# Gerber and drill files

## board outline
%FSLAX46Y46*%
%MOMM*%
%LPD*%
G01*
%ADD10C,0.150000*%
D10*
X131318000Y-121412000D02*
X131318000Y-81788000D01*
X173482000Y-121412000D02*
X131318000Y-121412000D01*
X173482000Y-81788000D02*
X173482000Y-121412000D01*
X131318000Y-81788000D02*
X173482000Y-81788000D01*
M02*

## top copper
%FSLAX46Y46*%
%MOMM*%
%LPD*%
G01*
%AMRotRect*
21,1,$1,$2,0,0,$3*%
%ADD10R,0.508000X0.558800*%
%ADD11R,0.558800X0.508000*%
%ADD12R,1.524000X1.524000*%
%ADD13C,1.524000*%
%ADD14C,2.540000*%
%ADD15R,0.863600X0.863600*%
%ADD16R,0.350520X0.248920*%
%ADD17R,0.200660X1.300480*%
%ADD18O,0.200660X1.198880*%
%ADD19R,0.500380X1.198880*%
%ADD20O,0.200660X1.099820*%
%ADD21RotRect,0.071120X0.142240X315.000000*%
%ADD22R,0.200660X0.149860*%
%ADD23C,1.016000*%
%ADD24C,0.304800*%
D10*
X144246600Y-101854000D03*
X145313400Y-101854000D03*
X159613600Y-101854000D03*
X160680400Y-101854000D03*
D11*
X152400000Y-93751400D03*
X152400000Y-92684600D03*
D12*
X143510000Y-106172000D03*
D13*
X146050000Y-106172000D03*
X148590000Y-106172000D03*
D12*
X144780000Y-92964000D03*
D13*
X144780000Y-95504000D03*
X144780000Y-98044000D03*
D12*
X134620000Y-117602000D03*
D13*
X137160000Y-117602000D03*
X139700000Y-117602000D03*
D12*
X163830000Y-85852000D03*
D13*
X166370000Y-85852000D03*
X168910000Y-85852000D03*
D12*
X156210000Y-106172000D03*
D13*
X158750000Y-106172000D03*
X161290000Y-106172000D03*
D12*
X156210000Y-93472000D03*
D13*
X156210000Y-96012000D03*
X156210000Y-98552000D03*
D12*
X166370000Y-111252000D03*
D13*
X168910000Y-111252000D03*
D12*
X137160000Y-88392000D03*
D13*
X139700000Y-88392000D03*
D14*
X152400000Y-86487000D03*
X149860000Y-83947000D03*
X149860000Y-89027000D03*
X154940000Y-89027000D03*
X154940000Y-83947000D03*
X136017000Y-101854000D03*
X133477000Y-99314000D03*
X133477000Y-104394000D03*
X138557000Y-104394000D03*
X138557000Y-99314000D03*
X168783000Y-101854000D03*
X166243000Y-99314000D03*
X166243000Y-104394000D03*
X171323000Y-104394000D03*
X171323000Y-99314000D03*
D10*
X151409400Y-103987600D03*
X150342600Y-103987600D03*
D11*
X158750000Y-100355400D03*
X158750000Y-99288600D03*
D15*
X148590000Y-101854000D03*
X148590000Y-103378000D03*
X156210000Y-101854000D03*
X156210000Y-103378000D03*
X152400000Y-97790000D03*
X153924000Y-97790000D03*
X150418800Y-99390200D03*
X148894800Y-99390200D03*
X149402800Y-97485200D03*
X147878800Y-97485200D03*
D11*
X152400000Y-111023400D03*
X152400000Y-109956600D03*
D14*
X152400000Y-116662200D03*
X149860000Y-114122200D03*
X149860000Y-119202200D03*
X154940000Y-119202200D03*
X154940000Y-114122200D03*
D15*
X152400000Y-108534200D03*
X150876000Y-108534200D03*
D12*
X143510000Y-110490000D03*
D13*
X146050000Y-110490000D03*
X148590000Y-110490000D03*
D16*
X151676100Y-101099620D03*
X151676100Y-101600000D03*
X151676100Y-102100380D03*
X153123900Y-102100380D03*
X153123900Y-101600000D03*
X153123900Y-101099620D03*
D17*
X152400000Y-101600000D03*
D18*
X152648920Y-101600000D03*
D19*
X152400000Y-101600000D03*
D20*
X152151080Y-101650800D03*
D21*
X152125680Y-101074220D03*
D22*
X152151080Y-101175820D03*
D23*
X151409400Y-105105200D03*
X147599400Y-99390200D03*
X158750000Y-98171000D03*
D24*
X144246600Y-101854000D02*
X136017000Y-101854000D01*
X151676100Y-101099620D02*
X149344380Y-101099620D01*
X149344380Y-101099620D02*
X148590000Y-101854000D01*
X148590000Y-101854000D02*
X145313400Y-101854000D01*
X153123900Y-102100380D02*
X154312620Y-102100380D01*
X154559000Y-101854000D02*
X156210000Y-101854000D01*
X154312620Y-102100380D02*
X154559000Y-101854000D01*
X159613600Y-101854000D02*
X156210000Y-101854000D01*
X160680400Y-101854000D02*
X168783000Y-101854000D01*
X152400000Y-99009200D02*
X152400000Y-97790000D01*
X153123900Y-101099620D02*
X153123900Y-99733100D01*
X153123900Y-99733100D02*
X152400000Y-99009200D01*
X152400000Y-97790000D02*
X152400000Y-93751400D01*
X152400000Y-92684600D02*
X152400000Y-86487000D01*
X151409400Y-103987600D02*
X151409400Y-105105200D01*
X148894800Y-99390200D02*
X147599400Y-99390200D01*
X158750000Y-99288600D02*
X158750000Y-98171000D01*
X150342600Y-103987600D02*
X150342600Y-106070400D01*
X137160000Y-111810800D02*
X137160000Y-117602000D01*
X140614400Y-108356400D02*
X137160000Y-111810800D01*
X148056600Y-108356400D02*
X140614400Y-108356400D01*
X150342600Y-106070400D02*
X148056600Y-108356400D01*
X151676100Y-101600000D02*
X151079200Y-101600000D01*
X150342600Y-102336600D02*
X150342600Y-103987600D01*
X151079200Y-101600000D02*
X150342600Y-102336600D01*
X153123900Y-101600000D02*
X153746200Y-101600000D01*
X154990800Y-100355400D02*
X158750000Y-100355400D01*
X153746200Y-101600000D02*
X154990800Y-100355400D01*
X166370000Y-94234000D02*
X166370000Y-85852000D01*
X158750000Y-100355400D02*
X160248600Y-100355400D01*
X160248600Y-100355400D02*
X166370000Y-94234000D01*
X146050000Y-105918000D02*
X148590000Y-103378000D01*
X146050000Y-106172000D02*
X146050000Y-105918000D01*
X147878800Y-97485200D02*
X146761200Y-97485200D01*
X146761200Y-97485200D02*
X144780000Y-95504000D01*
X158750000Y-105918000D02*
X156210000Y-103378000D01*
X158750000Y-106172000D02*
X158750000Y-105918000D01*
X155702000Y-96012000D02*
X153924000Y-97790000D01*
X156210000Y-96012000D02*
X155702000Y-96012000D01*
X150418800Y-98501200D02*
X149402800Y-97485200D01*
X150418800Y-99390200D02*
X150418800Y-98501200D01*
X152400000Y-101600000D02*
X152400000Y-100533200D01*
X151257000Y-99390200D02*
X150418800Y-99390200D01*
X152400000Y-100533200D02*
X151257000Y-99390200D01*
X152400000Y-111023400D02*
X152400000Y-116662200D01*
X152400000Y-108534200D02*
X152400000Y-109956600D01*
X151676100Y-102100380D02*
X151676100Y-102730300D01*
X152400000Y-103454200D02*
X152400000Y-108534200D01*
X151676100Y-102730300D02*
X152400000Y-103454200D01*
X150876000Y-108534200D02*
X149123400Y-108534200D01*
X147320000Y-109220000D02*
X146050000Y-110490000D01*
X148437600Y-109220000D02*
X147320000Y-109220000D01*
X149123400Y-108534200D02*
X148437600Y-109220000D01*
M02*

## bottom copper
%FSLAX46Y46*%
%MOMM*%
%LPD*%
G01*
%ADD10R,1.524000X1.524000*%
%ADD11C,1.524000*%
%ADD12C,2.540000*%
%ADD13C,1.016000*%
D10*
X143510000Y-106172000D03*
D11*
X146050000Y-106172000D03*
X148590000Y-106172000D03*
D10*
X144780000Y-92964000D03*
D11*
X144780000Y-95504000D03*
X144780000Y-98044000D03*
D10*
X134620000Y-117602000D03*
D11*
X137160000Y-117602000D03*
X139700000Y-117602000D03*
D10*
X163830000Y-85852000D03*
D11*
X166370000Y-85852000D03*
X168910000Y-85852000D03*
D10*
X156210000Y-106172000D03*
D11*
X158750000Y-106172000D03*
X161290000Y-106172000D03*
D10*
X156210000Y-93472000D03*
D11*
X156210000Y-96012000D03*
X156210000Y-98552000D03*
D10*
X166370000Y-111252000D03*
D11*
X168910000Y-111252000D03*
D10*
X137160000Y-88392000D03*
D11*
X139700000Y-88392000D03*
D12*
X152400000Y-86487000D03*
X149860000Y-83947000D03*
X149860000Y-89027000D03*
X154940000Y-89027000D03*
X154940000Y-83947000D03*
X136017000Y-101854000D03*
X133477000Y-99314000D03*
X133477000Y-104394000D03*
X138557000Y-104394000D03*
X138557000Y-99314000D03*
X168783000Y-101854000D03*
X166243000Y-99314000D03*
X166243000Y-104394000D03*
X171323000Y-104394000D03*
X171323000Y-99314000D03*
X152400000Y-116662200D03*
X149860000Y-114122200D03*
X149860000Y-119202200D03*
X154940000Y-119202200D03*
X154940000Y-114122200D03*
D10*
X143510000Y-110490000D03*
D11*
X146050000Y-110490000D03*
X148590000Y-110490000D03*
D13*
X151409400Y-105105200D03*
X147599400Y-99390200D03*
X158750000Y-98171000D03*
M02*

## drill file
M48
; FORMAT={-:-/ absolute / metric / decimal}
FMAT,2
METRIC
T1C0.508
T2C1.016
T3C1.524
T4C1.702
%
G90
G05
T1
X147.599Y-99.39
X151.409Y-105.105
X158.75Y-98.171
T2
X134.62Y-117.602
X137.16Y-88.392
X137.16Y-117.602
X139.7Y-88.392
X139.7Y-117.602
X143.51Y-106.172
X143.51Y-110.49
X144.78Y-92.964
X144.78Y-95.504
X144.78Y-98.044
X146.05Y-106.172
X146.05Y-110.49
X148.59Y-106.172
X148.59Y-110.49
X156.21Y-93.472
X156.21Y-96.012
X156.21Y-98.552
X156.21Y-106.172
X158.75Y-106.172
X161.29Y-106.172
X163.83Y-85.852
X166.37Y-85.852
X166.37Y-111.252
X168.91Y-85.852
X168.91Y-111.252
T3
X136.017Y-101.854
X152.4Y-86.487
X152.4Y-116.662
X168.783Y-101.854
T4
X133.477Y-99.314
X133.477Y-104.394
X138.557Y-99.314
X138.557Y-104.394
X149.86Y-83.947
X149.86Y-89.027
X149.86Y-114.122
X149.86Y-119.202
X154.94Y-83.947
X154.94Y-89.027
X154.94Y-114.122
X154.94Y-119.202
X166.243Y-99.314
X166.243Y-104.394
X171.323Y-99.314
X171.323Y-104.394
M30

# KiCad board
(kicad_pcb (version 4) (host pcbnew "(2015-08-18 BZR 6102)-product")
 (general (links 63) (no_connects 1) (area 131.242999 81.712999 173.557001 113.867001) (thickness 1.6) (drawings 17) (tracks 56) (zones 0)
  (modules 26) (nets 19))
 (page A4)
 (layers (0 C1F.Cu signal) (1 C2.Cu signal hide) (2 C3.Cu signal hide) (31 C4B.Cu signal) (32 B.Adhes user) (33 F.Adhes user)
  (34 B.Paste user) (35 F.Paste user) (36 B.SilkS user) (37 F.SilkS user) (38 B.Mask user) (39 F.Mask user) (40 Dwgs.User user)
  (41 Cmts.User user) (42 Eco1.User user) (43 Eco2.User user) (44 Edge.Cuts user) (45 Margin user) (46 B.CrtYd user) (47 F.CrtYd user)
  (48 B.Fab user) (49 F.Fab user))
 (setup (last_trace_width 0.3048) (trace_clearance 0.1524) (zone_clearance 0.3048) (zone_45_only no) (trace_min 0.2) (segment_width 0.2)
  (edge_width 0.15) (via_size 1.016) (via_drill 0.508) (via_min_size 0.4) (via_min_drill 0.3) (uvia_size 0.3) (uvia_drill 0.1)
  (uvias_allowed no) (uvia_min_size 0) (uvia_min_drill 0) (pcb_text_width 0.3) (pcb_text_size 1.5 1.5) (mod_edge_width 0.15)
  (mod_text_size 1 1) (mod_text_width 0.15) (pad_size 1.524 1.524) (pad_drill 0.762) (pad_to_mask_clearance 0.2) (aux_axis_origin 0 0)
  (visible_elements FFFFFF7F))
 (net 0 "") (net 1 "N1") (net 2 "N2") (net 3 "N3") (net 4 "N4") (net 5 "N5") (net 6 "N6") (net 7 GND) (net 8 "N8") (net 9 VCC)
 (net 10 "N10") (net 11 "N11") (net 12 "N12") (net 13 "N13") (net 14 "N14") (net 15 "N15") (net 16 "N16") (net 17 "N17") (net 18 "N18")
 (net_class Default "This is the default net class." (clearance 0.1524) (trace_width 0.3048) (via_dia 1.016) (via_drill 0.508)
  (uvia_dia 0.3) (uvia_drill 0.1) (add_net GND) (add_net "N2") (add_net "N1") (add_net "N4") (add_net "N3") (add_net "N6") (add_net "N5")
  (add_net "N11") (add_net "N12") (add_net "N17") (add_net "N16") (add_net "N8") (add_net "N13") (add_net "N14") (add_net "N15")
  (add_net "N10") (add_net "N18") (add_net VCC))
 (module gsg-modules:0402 (layer C1F.Cu) (at 144.78 101.854 180) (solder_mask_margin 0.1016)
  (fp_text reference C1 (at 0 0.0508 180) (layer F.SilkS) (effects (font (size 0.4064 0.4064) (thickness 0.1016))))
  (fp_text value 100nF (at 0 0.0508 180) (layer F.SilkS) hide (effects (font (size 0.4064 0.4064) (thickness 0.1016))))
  (pad 2 smd rect (at 0.5334 0 180) (size 0.508 0.5588) (layers C1F.Cu F.Paste F.Mask) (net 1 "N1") (solder_mask_margin 0.1016))
  (pad 1 smd rect (at -0.5334 0 180) (size 0.508 0.5588) (layers C1F.Cu F.Paste F.Mask) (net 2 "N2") (solder_mask_margin 0.1016)))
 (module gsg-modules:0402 (layer C1F.Cu) (at 160.147 101.854 180) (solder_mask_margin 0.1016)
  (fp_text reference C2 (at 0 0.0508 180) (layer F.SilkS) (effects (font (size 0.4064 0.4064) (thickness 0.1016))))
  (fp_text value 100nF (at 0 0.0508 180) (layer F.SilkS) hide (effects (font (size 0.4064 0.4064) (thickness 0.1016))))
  (pad 2 smd rect (at 0.5334 0 180) (size 0.508 0.5588) (layers C1F.Cu F.Paste F.Mask) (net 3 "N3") (solder_mask_margin 0.1016))
  (pad 1 smd rect (at -0.5334 0 180) (size 0.508 0.5588) (layers C1F.Cu F.Paste F.Mask) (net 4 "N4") (solder_mask_margin 0.1016)))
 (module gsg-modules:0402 (layer C1F.Cu) (at 152.4 93.218 270) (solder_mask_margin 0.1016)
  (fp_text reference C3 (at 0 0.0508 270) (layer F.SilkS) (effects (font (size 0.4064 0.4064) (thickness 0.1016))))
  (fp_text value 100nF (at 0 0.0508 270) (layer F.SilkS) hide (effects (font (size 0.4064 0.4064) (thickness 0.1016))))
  (pad 2 smd rect (at 0.5334 0 270) (size 0.508 0.5588) (layers C1F.Cu F.Paste F.Mask) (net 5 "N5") (solder_mask_margin 0.1016))
  (pad 1 smd rect (at -0.5334 0 270) (size 0.508 0.5588) (layers C1F.Cu F.Paste F.Mask) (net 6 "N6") (solder_mask_margin 0.1016)))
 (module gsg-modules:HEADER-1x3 (layer C1F.Cu) (at 146.05 106.172)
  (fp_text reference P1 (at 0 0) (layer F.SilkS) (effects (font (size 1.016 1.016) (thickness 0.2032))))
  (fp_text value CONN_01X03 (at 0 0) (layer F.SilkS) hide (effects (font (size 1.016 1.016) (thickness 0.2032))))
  (pad 1 thru_hole rect (at -2.54 0) (size 1.524 1.524) (drill 1.016) (layers *.Cu *.Mask F.SilkS) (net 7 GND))
  (pad 2 thru_hole circle (at 0 0) (size 1.524 1.524) (drill 1.016) (layers *.Cu *.Mask F.SilkS) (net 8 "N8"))
  (pad 3 thru_hole circle (at 2.54 0) (size 1.524 1.524) (drill 1.016) (layers *.Cu *.Mask F.SilkS) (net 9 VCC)))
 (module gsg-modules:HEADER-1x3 (layer C1F.Cu) (at 144.78 95.504 270)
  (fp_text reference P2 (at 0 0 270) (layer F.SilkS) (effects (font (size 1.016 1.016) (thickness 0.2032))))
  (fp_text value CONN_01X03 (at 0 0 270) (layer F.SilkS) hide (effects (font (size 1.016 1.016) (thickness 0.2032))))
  (pad 1 thru_hole rect (at -2.54 0 270) (size 1.524 1.524) (drill 1.016) (layers *.Cu *.Mask F.SilkS) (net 7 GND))
  (pad 2 thru_hole circle (at 0 0 270) (size 1.524 1.524) (drill 1.016) (layers *.Cu *.Mask F.SilkS) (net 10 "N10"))
  (pad 3 thru_hole circle (at 2.54 0 270) (size 1.524 1.524) (drill 1.016) (layers *.Cu *.Mask F.SilkS) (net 9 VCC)))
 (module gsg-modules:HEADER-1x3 (layer C1F.Cu) (at 137.16 117.602)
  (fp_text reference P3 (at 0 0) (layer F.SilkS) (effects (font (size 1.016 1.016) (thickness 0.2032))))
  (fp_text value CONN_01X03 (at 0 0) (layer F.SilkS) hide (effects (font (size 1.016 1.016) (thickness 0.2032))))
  (pad 1 thru_hole rect (at -2.54 0) (size 1.524 1.524) (drill 1.016) (layers *.Cu *.Mask F.SilkS) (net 7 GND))
  (pad 2 thru_hole circle (at 0 0) (size 1.524 1.524) (drill 1.016) (layers *.Cu *.Mask F.SilkS) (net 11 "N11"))
  (pad 3 thru_hole circle (at 2.54 0) (size 1.524 1.524) (drill 1.016) (layers *.Cu *.Mask F.SilkS) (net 9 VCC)))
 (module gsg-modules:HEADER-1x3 (layer C1F.Cu) (at 166.37 85.852)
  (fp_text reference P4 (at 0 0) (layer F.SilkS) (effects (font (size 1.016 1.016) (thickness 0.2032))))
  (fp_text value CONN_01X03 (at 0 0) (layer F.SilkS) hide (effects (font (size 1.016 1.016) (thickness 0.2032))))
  (pad 1 thru_hole rect (at -2.54 0) (size 1.524 1.524) (drill 1.016) (layers *.Cu *.Mask F.SilkS) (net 7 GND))
  (pad 2 thru_hole circle (at 0 0) (size 1.524 1.524) (drill 1.016) (layers *.Cu *.Mask F.SilkS) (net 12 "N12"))
  (pad 3 thru_hole circle (at 2.54 0) (size 1.524 1.524) (drill 1.016) (layers *.Cu *.Mask F.SilkS) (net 9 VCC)))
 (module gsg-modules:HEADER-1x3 (layer C1F.Cu) (at 158.75 106.172)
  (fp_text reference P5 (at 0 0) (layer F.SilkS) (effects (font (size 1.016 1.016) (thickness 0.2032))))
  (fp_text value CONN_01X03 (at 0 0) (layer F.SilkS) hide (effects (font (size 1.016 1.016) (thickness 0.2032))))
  (pad 1 thru_hole rect (at -2.54 0) (size 1.524 1.524) (drill 1.016) (layers *.Cu *.Mask F.SilkS) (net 7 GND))
  (pad 2 thru_hole circle (at 0 0) (size 1.524 1.524) (drill 1.016) (layers *.Cu *.Mask F.SilkS) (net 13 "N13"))
  (pad 3 thru_hole circle (at 2.54 0) (size 1.524 1.524) (drill 1.016) (layers *.Cu *.Mask F.SilkS) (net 9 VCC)))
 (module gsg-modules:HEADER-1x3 (layer C1F.Cu) (at 156.21 96.012 270)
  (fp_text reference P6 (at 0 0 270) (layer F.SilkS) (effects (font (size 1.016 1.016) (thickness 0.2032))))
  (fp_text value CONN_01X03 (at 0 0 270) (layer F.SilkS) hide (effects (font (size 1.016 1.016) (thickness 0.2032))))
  (pad 1 thru_hole rect (at -2.54 0 270) (size 1.524 1.524) (drill 1.016) (layers *.Cu *.Mask F.SilkS) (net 7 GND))
  (pad 2 thru_hole circle (at 0 0 270) (size 1.524 1.524) (drill 1.016) (layers *.Cu *.Mask F.SilkS) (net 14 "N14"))
  (pad 3 thru_hole circle (at 2.54 0 270) (size 1.524 1.524) (drill 1.016) (layers *.Cu *.Mask F.SilkS) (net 9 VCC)))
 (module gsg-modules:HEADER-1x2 (layer C1F.Cu) (at 167.64 111.252)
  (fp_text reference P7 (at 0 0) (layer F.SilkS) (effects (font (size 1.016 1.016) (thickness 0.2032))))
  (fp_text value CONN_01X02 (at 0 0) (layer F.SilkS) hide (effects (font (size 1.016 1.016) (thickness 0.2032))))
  (pad 1 thru_hole rect (at -1.27 0) (size 1.524 1.524) (drill 1.016) (layers *.Cu *.Mask F.SilkS) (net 9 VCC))
  (pad 2 thru_hole circle (at 1.27 0) (size 1.524 1.524) (drill 1.016) (layers *.Cu *.Mask F.SilkS) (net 9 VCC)))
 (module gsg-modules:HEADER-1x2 (layer C1F.Cu) (at 138.43 88.392)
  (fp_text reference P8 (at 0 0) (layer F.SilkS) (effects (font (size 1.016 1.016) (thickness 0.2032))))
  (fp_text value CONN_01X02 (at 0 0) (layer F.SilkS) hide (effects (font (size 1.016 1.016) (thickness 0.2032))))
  (pad 1 thru_hole rect (at -1.27 0) (size 1.524 1.524) (drill 1.016) (layers *.Cu *.Mask F.SilkS) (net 7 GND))
  (pad 2 thru_hole circle (at 1.27 0) (size 1.524 1.524) (drill 1.016) (layers *.Cu *.Mask F.SilkS) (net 7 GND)))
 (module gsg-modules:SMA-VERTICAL (layer C1F.Cu) (at 152.4 86.487)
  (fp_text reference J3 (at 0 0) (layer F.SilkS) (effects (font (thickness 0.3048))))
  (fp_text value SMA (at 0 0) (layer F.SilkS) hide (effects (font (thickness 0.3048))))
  (pad 1 thru_hole circle (at 0 0) (size 2.54 2.54) (drill 1.524) (layers *.Cu *.Mask F.SilkS) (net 6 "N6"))
  (pad 2 thru_hole circle (at -2.54 -2.54) (size 2.54 2.54) (drill 1.7018) (layers *.Cu *.Mask F.SilkS) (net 7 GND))
  (pad 2 thru_hole circle (at -2.54 2.54) (size 2.54 2.54) (drill 1.7018) (layers *.Cu *.Mask F.SilkS) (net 7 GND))
  (pad 2 thru_hole circle (at 2.54 2.54) (size 2.54 2.54) (drill 1.7018) (layers *.Cu *.Mask F.SilkS) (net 7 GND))
  (pad 2 thru_hole circle (at 2.54 -2.54) (size 2.54 2.54) (drill 1.7018) (layers *.Cu *.Mask F.SilkS) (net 7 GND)))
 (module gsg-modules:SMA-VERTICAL (layer C1F.Cu) (at 136.017 101.854)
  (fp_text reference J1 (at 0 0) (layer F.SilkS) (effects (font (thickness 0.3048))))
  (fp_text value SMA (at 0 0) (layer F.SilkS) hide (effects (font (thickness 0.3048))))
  (pad 1 thru_hole circle (at 0 0) (size 2.54 2.54) (drill 1.524) (layers *.Cu *.Mask F.SilkS) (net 1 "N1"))
  (pad 2 thru_hole circle (at -2.54 -2.54) (size 2.54 2.54) (drill 1.7018) (layers *.Cu *.Mask F.SilkS) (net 7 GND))
  (pad 2 thru_hole circle (at -2.54 2.54) (size 2.54 2.54) (drill 1.7018) (layers *.Cu *.Mask F.SilkS) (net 7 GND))
  (pad 2 thru_hole circle (at 2.54 2.54) (size 2.54 2.54) (drill 1.7018) (layers *.Cu *.Mask F.SilkS) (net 7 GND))
  (pad 2 thru_hole circle (at 2.54 -2.54) (size 2.54 2.54) (drill 1.7018) (layers *.Cu *.Mask F.SilkS) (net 7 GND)))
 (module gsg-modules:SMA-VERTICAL (layer C1F.Cu) (at 168.783 101.854)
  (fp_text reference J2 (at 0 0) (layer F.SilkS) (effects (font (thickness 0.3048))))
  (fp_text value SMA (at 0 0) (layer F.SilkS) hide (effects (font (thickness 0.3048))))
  (pad 1 thru_hole circle (at 0 0) (size 2.54 2.54) (drill 1.524) (layers *.Cu *.Mask F.SilkS) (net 4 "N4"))
  (pad 2 thru_hole circle (at -2.54 -2.54) (size 2.54 2.54) (drill 1.7018) (layers *.Cu *.Mask F.SilkS) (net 7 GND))
  (pad 2 thru_hole circle (at -2.54 2.54) (size 2.54 2.54) (drill 1.7018) (layers *.Cu *.Mask F.SilkS) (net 7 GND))
  (pad 2 thru_hole circle (at 2.54 2.54) (size 2.54 2.54) (drill 1.7018) (layers *.Cu *.Mask F.SilkS) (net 7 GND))
  (pad 2 thru_hole circle (at 2.54 -2.54) (size 2.54 2.54) (drill 1.7018) (layers *.Cu *.Mask F.SilkS) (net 7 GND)))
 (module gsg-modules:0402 (layer C1F.Cu) (at 150.876 103.9876) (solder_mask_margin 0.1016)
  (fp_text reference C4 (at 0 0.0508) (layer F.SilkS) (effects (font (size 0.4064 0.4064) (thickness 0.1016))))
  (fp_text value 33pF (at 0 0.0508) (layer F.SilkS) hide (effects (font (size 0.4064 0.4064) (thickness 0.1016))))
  (pad 2 smd rect (at 0.5334 0) (size 0.508 0.5588) (layers C1F.Cu F.Paste F.Mask) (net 7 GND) (solder_mask_margin 0.1016))
  (pad 1 smd rect (at -0.5334 0) (size 0.508 0.5588) (layers C1F.Cu F.Paste F.Mask) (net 11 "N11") (solder_mask_margin 0.1016)))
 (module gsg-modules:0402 (layer C1F.Cu) (at 158.75 99.822 270) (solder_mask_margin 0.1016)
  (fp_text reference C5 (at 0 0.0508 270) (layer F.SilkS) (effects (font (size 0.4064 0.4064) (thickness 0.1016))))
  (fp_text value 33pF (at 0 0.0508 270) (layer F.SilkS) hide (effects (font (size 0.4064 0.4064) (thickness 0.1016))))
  (pad 2 smd rect (at 0.5334 0 270) (size 0.508 0.5588) (layers C1F.Cu F.Paste F.Mask) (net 12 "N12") (solder_mask_margin 0.1016))
  (pad 1 smd rect (at -0.5334 0 270) (size 0.508 0.5588) (layers C1F.Cu F.Paste F.Mask) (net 7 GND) (solder_mask_margin 0.1016)))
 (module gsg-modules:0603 (layer C1F.Cu) (at 148.59 102.616 90) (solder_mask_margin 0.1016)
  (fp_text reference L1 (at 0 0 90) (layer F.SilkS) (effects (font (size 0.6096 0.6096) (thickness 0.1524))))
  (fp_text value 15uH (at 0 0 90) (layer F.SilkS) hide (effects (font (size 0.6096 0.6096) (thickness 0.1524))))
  (pad 2 smd rect (at 0.762 0 90) (size 0.8636 0.8636) (layers C1F.Cu F.Paste F.Mask) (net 2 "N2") (solder_mask_margin 0.1016)
   (clearance 0.1778))
  (pad 1 smd rect (at -0.762 0 90) (size 0.8636 0.8636) (layers C1F.Cu F.Paste F.Mask) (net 8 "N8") (solder_mask_margin 0.1016)
   (clearance 0.1778)))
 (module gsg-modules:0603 (layer C1F.Cu) (at 156.21 102.616 90) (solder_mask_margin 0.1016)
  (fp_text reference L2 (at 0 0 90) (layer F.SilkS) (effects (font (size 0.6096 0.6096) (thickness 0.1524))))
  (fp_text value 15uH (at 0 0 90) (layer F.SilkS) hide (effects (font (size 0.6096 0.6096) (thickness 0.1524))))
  (pad 2 smd rect (at 0.762 0 90) (size 0.8636 0.8636) (layers C1F.Cu F.Paste F.Mask) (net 3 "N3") (solder_mask_margin 0.1016)
   (clearance 0.1778))
  (pad 1 smd rect (at -0.762 0 90) (size 0.8636 0.8636) (layers C1F.Cu F.Paste F.Mask) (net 13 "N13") (solder_mask_margin 0.1016)
   (clearance 0.1778)))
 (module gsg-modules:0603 (layer C1F.Cu) (at 153.162 97.79 180) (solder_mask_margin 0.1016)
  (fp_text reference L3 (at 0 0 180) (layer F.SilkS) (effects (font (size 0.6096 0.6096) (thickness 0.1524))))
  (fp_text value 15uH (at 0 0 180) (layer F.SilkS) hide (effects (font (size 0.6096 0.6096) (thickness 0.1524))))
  (pad 2 smd rect (at 0.762 0 180) (size 0.8636 0.8636) (layers C1F.Cu F.Paste F.Mask) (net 5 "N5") (solder_mask_margin 0.1016)
   (clearance 0.1778))
  (pad 1 smd rect (at -0.762 0 180) (size 0.8636 0.8636) (layers C1F.Cu F.Paste F.Mask) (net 14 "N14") (solder_mask_margin 0.1016)
   (clearance 0.1778)))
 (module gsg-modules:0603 (layer C1F.Cu) (at 149.6568 99.3902) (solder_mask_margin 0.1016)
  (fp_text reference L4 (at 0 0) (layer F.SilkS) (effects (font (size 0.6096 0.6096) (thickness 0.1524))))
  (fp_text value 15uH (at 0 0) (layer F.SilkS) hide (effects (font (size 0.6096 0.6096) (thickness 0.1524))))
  (pad 2 smd rect (at 0.762 0) (size 0.8636 0.8636) (layers C1F.Cu F.Paste F.Mask) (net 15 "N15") (solder_mask_margin 0.1016)
   (clearance 0.1778))
  (pad 1 smd rect (at -0.762 0) (size 0.8636 0.8636) (layers C1F.Cu F.Paste F.Mask) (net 7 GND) (solder_mask_margin 0.1016)
   (clearance 0.1778)))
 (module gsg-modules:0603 (layer C1F.Cu) (at 148.6408 97.4852) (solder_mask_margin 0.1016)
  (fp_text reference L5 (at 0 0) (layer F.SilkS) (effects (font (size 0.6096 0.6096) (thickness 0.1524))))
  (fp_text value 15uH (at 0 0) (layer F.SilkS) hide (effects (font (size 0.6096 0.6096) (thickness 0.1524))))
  (pad 2 smd rect (at 0.762 0) (size 0.8636 0.8636) (layers C1F.Cu F.Paste F.Mask) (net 15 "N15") (solder_mask_margin 0.1016)
   (clearance 0.1778))
  (pad 1 smd rect (at -0.762 0) (size 0.8636 0.8636) (layers C1F.Cu F.Paste F.Mask) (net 10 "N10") (solder_mask_margin 0.1016)
   (clearance 0.1778)))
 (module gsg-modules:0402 (layer C1F.Cu) (at 152.4 110.49 270) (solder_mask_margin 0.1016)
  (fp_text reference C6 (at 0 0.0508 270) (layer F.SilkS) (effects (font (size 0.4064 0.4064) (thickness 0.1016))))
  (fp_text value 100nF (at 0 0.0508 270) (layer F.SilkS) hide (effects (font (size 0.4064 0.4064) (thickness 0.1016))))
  (pad 2 smd rect (at 0.5334 0 270) (size 0.508 0.5588) (layers C1F.Cu F.Paste F.Mask) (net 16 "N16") (solder_mask_margin 0.1016))
  (pad 1 smd rect (at -0.5334 0 270) (size 0.508 0.5588) (layers C1F.Cu F.Paste F.Mask) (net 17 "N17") (solder_mask_margin 0.1016)))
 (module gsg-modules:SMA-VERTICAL (layer C1F.Cu) (at 152.4 116.6622)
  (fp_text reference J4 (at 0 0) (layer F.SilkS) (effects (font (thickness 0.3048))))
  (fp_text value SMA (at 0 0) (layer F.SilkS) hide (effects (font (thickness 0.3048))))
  (pad 1 thru_hole circle (at 0 0) (size 2.54 2.54) (drill 1.524) (layers *.Cu *.Mask F.SilkS) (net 16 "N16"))
  (pad 2 thru_hole circle (at -2.54 -2.54) (size 2.54 2.54) (drill 1.7018) (layers *.Cu *.Mask F.SilkS) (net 7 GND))
  (pad 2 thru_hole circle (at -2.54 2.54) (size 2.54 2.54) (drill 1.7018) (layers *.Cu *.Mask F.SilkS) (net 7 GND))
  (pad 2 thru_hole circle (at 2.54 2.54) (size 2.54 2.54) (drill 1.7018) (layers *.Cu *.Mask F.SilkS) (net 7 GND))
  (pad 2 thru_hole circle (at 2.54 -2.54) (size 2.54 2.54) (drill 1.7018) (layers *.Cu *.Mask F.SilkS) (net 7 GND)))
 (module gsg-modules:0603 (layer C1F.Cu) (at 151.638 108.5342) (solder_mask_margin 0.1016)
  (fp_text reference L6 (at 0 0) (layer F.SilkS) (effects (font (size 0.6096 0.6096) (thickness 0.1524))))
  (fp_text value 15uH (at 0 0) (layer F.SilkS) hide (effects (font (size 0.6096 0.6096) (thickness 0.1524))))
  (pad 2 smd rect (at 0.762 0) (size 0.8636 0.8636) (layers C1F.Cu F.Paste F.Mask) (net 17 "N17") (solder_mask_margin 0.1016)
   (clearance 0.1778))
  (pad 1 smd rect (at -0.762 0) (size 0.8636 0.8636) (layers C1F.Cu F.Paste F.Mask) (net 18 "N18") (solder_mask_margin 0.1016)
   (clearance 0.1778)))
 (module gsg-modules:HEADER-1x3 (layer C1F.Cu) (at 146.05 110.49)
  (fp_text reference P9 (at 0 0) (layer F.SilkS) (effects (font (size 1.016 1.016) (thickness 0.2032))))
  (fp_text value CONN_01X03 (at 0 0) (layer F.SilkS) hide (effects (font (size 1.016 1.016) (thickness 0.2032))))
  (pad 1 thru_hole rect (at -2.54 0) (size 1.524 1.524) (drill 1.016) (layers *.Cu *.Mask F.SilkS) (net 7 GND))
  (pad 2 thru_hole circle (at 0 0) (size 1.524 1.524) (drill 1.016) (layers *.Cu *.Mask F.SilkS) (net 18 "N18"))
  (pad 3 thru_hole circle (at 2.54 0) (size 1.524 1.524) (drill 1.016) (layers *.Cu *.Mask F.SilkS) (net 9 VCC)))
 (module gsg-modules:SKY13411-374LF (layer C1F.Cu) (at 152.4 101.6) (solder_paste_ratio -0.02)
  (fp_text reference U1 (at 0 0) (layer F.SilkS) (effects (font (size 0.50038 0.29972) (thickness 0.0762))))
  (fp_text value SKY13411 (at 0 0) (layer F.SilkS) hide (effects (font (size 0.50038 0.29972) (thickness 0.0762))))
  (pad 1 smd rect (at -0.7239 -0.50038) (size 0.35052 0.24892) (layers C1F.Cu F.Paste F.Mask) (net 2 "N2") (die_length -2147.483648))
  (pad 2 smd rect (at -0.7239 0) (size 0.35052 0.24892) (layers C1F.Cu F.Paste F.Mask) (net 11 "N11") (die_length -2147.483648))
  (pad 3 smd rect (at -0.7239 0.50038) (size 0.35052 0.24892) (layers C1F.Cu F.Paste F.Mask) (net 17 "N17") (die_length -2147.483648))
  (pad 4 smd rect (at 0.7239 0.50038) (size 0.35052 0.24892) (layers C1F.Cu F.Paste F.Mask) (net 3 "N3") (die_length 0.0508))
  (pad 5 smd rect (at 0.7239 0) (size 0.35052 0.24892) (layers C1F.Cu F.Paste F.Mask) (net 12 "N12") (die_length 10.53846))
  (pad 6 smd rect (at 0.7239 -0.50038) (size 0.35052 0.24892) (layers C1F.Cu F.Paste F.Mask) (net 5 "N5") (die_length -2147.483648))
  (pad 0 smd rect (at 0 0) (size 0.20066 1.30048) (layers C1F.Cu F.Paste F.Mask) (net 15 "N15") (die_length -2147.483648))
  (pad 0 smd oval (at 0.24892 0) (size 0.20066 1.19888) (layers C1F.Cu F.Paste F.Mask) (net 15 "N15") (die_length -2147.483648))
  (pad 0 smd rect (at 0 0) (size 0.50038 1.19888) (layers C1F.Cu F.Paste F.Mask) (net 15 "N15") (die_length -2147.483648))
  (pad 0 smd oval (at -0.24892 0.0508) (size 0.20066 1.09982) (layers C1F.Cu F.Paste F.Mask) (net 15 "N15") (die_length -2147.483648))
  (pad 0 smd rect (at -0.27432 -0.52578 315) (size 0.07112 0.14224) (layers C1F.Cu F.Paste F.Mask) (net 15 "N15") (die_length -2147.483648))
  (pad 0 smd rect (at -0.24892 -0.42418) (size 0.20066 0.14986) (layers C1F.Cu F.Paste F.Mask) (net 15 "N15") (die_length -2147.483648)))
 (gr_line (start 131.318 121.412) (end 131.318 81.788) (angle 90) (layer Edge.Cuts) (width 0.15))
 (gr_line (start 173.482 121.412) (end 131.318 121.412) (angle 90) (layer Edge.Cuts) (width 0.15))
 (gr_line (start 173.482 81.788) (end 173.482 121.412) (angle 90) (layer Edge.Cuts) (width 0.15))
 (gr_line (start 131.318 81.788) (end 173.482 81.788) (angle 90) (layer Edge.Cuts) (width 0.15))
 (segment (start 144.2466 101.854) (end 136.017 101.854) (width 0.3048) (layer C1F.Cu) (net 1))
 (segment (start 151.6761 101.09962) (end 149.34438 101.09962) (width 0.3048) (layer C1F.Cu) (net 2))
 (segment (start 149.34438 101.09962) (end 148.59 101.854) (width 0.3048) (layer C1F.Cu) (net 2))
 (segment (start 148.59 101.854) (end 145.3134 101.854) (width 0.3048) (layer C1F.Cu) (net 2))
 (segment (start 153.1239 102.10038) (end 154.31262 102.10038) (width 0.3048) (layer C1F.Cu) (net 3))
 (segment (start 154.559 101.854) (end 156.21 101.854) (width 0.3048) (layer C1F.Cu) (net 3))
 (segment (start 154.31262 102.10038) (end 154.559 101.854) (width 0.3048) (layer C1F.Cu) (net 3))
 (segment (start 159.6136 101.854) (end 156.21 101.854) (width 0.3048) (layer C1F.Cu) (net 3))
 (segment (start 160.6804 101.854) (end 168.783 101.854) (width 0.3048) (layer C1F.Cu) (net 4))
 (segment (start 152.4 99.0092) (end 152.4 97.79) (width 0.3048) (layer C1F.Cu) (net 5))
 (segment (start 153.1239 101.09962) (end 153.1239 99.7331) (width 0.3048) (layer C1F.Cu) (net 5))
 (segment (start 153.1239 99.7331) (end 152.4 99.0092) (width 0.3048) (layer C1F.Cu) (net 5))
 (segment (start 152.4 97.79) (end 152.4 93.7514) (width 0.3048) (layer C1F.Cu) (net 5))
 (segment (start 152.4 92.6846) (end 152.4 86.487) (width 0.3048) (layer C1F.Cu) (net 6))
 (segment (start 151.4094 103.9876) (end 151.4094 105.1052) (width 0.3048) (layer C1F.Cu) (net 7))
 (via (at 151.4094 105.1052) (size 1.016) (drill 0.508) (layers C1F.Cu C4B.Cu) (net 7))
 (segment (start 148.8948 99.3902) (end 147.5994 99.3902) (width 0.3048) (layer C1F.Cu) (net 7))
 (via (at 147.5994 99.3902) (size 1.016) (drill 0.508) (layers C1F.Cu C4B.Cu) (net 7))
 (segment (start 158.75 99.2886) (end 158.75 98.171) (width 0.3048) (layer C1F.Cu) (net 7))
 (via (at 158.75 98.171) (size 1.016) (drill 0.508) (layers C1F.Cu C4B.Cu) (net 7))
 (segment (start 150.3426 103.9876) (end 150.3426 106.0704) (width 0.3048) (layer C1F.Cu) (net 11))
 (segment (start 137.16 111.8108) (end 137.16 117.602) (width 0.3048) (layer C1F.Cu) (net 11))
 (segment (start 140.6144 108.3564) (end 137.16 111.8108) (width 0.3048) (layer C1F.Cu) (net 11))
 (segment (start 148.0566 108.3564) (end 140.6144 108.3564) (width 0.3048) (layer C1F.Cu) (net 11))
 (segment (start 150.3426 106.0704) (end 148.0566 108.3564) (width 0.3048) (layer C1F.Cu) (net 11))
 (segment (start 151.6761 101.6) (end 151.0792 101.6) (width 0.3048) (layer C1F.Cu) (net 11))
 (segment (start 150.3426 102.3366) (end 150.3426 103.9876) (width 0.3048) (layer C1F.Cu) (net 11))
 (segment (start 151.0792 101.6) (end 150.3426 102.3366) (width 0.3048) (layer C1F.Cu) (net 11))
 (segment (start 153.1239 101.6) (end 153.7462 101.6) (width 0.3048) (layer C1F.Cu) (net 12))
 (segment (start 154.9908 100.3554) (end 158.75 100.3554) (width 0.3048) (layer C1F.Cu) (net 12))
 (segment (start 153.7462 101.6) (end 154.9908 100.3554) (width 0.3048) (layer C1F.Cu) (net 12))
 (segment (start 166.37 94.234) (end 166.37 85.852) (width 0.3048) (layer C1F.Cu) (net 12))
 (segment (start 158.75 100.3554) (end 160.2486 100.3554) (width 0.3048) (layer C1F.Cu) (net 12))
 (segment (start 160.2486 100.3554) (end 166.37 94.234) (width 0.3048) (layer C1F.Cu) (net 12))
 (segment (start 146.05 105.918) (end 148.59 103.378) (width 0.3048) (layer C1F.Cu) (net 8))
 (segment (start 146.05 106.172) (end 146.05 105.918) (width 0.3048) (layer C1F.Cu) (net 8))
 (segment (start 147.8788 97.4852) (end 146.7612 97.4852) (width 0.3048) (layer C1F.Cu) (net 10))
 (segment (start 146.7612 97.4852) (end 144.78 95.504) (width 0.3048) (layer C1F.Cu) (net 10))
 (segment (start 158.75 105.918) (end 156.21 103.378) (width 0.3048) (layer C1F.Cu) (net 13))
 (segment (start 158.75 106.172) (end 158.75 105.918) (width 0.3048) (layer C1F.Cu) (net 13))
 (segment (start 155.702 96.012) (end 153.924 97.79) (width 0.3048) (layer C1F.Cu) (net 14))
 (segment (start 156.21 96.012) (end 155.702 96.012) (width 0.3048) (layer C1F.Cu) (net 14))
 (segment (start 150.4188 98.5012) (end 149.4028 97.4852) (width 0.3048) (layer C1F.Cu) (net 15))
 (segment (start 150.4188 99.3902) (end 150.4188 98.5012) (width 0.3048) (layer C1F.Cu) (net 15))
 (segment (start 152.4 101.6) (end 152.4 100.5332) (width 0.3048) (layer C1F.Cu) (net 15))
 (segment (start 151.257 99.3902) (end 150.4188 99.3902) (width 0.3048) (layer C1F.Cu) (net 15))
 (segment (start 152.4 100.5332) (end 151.257 99.3902) (width 0.3048) (layer C1F.Cu) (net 15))
 (segment (start 152.4 111.0234) (end 152.4 116.6622) (width 0.3048) (layer C1F.Cu) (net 16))
 (segment (start 152.4 108.5342) (end 152.4 109.9566) (width 0.3048) (layer C1F.Cu) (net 17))
 (segment (start 151.6761 102.10038) (end 151.6761 102.7303) (width 0.3048) (layer C1F.Cu) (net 17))
 (segment (start 152.4 103.4542) (end 152.4 108.5342) (width 0.3048) (layer C1F.Cu) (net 17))
 (segment (start 151.6761 102.7303) (end 152.4 103.4542) (width 0.3048) (layer C1F.Cu) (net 17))
 (segment (start 150.876 108.5342) (end 149.1234 108.5342) (width 0.3048) (layer C1F.Cu) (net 18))
 (segment (start 147.32 109.22) (end 146.05 110.49) (width 0.3048) (layer C1F.Cu) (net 18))
 (segment (start 148.4376 109.22) (end 147.32 109.22) (width 0.3048) (layer C1F.Cu) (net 18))
 (segment (start 149.1234 108.5342) (end 148.4376 109.22) (width 0.3048) (layer C1F.Cu) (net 18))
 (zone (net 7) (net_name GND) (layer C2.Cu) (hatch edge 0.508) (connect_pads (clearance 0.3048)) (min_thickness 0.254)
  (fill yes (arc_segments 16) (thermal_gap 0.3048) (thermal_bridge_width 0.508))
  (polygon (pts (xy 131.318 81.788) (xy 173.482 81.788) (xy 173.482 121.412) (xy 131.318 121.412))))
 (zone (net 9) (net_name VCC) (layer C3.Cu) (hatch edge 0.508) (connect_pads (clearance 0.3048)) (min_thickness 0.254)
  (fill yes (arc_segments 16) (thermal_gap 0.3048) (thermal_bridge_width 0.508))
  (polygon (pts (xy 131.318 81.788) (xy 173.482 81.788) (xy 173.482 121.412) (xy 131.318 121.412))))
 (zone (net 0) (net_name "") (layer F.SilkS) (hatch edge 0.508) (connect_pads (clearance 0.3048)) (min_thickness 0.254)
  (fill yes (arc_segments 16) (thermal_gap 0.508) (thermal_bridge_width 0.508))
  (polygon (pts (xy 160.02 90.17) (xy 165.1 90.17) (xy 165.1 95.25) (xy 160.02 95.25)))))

